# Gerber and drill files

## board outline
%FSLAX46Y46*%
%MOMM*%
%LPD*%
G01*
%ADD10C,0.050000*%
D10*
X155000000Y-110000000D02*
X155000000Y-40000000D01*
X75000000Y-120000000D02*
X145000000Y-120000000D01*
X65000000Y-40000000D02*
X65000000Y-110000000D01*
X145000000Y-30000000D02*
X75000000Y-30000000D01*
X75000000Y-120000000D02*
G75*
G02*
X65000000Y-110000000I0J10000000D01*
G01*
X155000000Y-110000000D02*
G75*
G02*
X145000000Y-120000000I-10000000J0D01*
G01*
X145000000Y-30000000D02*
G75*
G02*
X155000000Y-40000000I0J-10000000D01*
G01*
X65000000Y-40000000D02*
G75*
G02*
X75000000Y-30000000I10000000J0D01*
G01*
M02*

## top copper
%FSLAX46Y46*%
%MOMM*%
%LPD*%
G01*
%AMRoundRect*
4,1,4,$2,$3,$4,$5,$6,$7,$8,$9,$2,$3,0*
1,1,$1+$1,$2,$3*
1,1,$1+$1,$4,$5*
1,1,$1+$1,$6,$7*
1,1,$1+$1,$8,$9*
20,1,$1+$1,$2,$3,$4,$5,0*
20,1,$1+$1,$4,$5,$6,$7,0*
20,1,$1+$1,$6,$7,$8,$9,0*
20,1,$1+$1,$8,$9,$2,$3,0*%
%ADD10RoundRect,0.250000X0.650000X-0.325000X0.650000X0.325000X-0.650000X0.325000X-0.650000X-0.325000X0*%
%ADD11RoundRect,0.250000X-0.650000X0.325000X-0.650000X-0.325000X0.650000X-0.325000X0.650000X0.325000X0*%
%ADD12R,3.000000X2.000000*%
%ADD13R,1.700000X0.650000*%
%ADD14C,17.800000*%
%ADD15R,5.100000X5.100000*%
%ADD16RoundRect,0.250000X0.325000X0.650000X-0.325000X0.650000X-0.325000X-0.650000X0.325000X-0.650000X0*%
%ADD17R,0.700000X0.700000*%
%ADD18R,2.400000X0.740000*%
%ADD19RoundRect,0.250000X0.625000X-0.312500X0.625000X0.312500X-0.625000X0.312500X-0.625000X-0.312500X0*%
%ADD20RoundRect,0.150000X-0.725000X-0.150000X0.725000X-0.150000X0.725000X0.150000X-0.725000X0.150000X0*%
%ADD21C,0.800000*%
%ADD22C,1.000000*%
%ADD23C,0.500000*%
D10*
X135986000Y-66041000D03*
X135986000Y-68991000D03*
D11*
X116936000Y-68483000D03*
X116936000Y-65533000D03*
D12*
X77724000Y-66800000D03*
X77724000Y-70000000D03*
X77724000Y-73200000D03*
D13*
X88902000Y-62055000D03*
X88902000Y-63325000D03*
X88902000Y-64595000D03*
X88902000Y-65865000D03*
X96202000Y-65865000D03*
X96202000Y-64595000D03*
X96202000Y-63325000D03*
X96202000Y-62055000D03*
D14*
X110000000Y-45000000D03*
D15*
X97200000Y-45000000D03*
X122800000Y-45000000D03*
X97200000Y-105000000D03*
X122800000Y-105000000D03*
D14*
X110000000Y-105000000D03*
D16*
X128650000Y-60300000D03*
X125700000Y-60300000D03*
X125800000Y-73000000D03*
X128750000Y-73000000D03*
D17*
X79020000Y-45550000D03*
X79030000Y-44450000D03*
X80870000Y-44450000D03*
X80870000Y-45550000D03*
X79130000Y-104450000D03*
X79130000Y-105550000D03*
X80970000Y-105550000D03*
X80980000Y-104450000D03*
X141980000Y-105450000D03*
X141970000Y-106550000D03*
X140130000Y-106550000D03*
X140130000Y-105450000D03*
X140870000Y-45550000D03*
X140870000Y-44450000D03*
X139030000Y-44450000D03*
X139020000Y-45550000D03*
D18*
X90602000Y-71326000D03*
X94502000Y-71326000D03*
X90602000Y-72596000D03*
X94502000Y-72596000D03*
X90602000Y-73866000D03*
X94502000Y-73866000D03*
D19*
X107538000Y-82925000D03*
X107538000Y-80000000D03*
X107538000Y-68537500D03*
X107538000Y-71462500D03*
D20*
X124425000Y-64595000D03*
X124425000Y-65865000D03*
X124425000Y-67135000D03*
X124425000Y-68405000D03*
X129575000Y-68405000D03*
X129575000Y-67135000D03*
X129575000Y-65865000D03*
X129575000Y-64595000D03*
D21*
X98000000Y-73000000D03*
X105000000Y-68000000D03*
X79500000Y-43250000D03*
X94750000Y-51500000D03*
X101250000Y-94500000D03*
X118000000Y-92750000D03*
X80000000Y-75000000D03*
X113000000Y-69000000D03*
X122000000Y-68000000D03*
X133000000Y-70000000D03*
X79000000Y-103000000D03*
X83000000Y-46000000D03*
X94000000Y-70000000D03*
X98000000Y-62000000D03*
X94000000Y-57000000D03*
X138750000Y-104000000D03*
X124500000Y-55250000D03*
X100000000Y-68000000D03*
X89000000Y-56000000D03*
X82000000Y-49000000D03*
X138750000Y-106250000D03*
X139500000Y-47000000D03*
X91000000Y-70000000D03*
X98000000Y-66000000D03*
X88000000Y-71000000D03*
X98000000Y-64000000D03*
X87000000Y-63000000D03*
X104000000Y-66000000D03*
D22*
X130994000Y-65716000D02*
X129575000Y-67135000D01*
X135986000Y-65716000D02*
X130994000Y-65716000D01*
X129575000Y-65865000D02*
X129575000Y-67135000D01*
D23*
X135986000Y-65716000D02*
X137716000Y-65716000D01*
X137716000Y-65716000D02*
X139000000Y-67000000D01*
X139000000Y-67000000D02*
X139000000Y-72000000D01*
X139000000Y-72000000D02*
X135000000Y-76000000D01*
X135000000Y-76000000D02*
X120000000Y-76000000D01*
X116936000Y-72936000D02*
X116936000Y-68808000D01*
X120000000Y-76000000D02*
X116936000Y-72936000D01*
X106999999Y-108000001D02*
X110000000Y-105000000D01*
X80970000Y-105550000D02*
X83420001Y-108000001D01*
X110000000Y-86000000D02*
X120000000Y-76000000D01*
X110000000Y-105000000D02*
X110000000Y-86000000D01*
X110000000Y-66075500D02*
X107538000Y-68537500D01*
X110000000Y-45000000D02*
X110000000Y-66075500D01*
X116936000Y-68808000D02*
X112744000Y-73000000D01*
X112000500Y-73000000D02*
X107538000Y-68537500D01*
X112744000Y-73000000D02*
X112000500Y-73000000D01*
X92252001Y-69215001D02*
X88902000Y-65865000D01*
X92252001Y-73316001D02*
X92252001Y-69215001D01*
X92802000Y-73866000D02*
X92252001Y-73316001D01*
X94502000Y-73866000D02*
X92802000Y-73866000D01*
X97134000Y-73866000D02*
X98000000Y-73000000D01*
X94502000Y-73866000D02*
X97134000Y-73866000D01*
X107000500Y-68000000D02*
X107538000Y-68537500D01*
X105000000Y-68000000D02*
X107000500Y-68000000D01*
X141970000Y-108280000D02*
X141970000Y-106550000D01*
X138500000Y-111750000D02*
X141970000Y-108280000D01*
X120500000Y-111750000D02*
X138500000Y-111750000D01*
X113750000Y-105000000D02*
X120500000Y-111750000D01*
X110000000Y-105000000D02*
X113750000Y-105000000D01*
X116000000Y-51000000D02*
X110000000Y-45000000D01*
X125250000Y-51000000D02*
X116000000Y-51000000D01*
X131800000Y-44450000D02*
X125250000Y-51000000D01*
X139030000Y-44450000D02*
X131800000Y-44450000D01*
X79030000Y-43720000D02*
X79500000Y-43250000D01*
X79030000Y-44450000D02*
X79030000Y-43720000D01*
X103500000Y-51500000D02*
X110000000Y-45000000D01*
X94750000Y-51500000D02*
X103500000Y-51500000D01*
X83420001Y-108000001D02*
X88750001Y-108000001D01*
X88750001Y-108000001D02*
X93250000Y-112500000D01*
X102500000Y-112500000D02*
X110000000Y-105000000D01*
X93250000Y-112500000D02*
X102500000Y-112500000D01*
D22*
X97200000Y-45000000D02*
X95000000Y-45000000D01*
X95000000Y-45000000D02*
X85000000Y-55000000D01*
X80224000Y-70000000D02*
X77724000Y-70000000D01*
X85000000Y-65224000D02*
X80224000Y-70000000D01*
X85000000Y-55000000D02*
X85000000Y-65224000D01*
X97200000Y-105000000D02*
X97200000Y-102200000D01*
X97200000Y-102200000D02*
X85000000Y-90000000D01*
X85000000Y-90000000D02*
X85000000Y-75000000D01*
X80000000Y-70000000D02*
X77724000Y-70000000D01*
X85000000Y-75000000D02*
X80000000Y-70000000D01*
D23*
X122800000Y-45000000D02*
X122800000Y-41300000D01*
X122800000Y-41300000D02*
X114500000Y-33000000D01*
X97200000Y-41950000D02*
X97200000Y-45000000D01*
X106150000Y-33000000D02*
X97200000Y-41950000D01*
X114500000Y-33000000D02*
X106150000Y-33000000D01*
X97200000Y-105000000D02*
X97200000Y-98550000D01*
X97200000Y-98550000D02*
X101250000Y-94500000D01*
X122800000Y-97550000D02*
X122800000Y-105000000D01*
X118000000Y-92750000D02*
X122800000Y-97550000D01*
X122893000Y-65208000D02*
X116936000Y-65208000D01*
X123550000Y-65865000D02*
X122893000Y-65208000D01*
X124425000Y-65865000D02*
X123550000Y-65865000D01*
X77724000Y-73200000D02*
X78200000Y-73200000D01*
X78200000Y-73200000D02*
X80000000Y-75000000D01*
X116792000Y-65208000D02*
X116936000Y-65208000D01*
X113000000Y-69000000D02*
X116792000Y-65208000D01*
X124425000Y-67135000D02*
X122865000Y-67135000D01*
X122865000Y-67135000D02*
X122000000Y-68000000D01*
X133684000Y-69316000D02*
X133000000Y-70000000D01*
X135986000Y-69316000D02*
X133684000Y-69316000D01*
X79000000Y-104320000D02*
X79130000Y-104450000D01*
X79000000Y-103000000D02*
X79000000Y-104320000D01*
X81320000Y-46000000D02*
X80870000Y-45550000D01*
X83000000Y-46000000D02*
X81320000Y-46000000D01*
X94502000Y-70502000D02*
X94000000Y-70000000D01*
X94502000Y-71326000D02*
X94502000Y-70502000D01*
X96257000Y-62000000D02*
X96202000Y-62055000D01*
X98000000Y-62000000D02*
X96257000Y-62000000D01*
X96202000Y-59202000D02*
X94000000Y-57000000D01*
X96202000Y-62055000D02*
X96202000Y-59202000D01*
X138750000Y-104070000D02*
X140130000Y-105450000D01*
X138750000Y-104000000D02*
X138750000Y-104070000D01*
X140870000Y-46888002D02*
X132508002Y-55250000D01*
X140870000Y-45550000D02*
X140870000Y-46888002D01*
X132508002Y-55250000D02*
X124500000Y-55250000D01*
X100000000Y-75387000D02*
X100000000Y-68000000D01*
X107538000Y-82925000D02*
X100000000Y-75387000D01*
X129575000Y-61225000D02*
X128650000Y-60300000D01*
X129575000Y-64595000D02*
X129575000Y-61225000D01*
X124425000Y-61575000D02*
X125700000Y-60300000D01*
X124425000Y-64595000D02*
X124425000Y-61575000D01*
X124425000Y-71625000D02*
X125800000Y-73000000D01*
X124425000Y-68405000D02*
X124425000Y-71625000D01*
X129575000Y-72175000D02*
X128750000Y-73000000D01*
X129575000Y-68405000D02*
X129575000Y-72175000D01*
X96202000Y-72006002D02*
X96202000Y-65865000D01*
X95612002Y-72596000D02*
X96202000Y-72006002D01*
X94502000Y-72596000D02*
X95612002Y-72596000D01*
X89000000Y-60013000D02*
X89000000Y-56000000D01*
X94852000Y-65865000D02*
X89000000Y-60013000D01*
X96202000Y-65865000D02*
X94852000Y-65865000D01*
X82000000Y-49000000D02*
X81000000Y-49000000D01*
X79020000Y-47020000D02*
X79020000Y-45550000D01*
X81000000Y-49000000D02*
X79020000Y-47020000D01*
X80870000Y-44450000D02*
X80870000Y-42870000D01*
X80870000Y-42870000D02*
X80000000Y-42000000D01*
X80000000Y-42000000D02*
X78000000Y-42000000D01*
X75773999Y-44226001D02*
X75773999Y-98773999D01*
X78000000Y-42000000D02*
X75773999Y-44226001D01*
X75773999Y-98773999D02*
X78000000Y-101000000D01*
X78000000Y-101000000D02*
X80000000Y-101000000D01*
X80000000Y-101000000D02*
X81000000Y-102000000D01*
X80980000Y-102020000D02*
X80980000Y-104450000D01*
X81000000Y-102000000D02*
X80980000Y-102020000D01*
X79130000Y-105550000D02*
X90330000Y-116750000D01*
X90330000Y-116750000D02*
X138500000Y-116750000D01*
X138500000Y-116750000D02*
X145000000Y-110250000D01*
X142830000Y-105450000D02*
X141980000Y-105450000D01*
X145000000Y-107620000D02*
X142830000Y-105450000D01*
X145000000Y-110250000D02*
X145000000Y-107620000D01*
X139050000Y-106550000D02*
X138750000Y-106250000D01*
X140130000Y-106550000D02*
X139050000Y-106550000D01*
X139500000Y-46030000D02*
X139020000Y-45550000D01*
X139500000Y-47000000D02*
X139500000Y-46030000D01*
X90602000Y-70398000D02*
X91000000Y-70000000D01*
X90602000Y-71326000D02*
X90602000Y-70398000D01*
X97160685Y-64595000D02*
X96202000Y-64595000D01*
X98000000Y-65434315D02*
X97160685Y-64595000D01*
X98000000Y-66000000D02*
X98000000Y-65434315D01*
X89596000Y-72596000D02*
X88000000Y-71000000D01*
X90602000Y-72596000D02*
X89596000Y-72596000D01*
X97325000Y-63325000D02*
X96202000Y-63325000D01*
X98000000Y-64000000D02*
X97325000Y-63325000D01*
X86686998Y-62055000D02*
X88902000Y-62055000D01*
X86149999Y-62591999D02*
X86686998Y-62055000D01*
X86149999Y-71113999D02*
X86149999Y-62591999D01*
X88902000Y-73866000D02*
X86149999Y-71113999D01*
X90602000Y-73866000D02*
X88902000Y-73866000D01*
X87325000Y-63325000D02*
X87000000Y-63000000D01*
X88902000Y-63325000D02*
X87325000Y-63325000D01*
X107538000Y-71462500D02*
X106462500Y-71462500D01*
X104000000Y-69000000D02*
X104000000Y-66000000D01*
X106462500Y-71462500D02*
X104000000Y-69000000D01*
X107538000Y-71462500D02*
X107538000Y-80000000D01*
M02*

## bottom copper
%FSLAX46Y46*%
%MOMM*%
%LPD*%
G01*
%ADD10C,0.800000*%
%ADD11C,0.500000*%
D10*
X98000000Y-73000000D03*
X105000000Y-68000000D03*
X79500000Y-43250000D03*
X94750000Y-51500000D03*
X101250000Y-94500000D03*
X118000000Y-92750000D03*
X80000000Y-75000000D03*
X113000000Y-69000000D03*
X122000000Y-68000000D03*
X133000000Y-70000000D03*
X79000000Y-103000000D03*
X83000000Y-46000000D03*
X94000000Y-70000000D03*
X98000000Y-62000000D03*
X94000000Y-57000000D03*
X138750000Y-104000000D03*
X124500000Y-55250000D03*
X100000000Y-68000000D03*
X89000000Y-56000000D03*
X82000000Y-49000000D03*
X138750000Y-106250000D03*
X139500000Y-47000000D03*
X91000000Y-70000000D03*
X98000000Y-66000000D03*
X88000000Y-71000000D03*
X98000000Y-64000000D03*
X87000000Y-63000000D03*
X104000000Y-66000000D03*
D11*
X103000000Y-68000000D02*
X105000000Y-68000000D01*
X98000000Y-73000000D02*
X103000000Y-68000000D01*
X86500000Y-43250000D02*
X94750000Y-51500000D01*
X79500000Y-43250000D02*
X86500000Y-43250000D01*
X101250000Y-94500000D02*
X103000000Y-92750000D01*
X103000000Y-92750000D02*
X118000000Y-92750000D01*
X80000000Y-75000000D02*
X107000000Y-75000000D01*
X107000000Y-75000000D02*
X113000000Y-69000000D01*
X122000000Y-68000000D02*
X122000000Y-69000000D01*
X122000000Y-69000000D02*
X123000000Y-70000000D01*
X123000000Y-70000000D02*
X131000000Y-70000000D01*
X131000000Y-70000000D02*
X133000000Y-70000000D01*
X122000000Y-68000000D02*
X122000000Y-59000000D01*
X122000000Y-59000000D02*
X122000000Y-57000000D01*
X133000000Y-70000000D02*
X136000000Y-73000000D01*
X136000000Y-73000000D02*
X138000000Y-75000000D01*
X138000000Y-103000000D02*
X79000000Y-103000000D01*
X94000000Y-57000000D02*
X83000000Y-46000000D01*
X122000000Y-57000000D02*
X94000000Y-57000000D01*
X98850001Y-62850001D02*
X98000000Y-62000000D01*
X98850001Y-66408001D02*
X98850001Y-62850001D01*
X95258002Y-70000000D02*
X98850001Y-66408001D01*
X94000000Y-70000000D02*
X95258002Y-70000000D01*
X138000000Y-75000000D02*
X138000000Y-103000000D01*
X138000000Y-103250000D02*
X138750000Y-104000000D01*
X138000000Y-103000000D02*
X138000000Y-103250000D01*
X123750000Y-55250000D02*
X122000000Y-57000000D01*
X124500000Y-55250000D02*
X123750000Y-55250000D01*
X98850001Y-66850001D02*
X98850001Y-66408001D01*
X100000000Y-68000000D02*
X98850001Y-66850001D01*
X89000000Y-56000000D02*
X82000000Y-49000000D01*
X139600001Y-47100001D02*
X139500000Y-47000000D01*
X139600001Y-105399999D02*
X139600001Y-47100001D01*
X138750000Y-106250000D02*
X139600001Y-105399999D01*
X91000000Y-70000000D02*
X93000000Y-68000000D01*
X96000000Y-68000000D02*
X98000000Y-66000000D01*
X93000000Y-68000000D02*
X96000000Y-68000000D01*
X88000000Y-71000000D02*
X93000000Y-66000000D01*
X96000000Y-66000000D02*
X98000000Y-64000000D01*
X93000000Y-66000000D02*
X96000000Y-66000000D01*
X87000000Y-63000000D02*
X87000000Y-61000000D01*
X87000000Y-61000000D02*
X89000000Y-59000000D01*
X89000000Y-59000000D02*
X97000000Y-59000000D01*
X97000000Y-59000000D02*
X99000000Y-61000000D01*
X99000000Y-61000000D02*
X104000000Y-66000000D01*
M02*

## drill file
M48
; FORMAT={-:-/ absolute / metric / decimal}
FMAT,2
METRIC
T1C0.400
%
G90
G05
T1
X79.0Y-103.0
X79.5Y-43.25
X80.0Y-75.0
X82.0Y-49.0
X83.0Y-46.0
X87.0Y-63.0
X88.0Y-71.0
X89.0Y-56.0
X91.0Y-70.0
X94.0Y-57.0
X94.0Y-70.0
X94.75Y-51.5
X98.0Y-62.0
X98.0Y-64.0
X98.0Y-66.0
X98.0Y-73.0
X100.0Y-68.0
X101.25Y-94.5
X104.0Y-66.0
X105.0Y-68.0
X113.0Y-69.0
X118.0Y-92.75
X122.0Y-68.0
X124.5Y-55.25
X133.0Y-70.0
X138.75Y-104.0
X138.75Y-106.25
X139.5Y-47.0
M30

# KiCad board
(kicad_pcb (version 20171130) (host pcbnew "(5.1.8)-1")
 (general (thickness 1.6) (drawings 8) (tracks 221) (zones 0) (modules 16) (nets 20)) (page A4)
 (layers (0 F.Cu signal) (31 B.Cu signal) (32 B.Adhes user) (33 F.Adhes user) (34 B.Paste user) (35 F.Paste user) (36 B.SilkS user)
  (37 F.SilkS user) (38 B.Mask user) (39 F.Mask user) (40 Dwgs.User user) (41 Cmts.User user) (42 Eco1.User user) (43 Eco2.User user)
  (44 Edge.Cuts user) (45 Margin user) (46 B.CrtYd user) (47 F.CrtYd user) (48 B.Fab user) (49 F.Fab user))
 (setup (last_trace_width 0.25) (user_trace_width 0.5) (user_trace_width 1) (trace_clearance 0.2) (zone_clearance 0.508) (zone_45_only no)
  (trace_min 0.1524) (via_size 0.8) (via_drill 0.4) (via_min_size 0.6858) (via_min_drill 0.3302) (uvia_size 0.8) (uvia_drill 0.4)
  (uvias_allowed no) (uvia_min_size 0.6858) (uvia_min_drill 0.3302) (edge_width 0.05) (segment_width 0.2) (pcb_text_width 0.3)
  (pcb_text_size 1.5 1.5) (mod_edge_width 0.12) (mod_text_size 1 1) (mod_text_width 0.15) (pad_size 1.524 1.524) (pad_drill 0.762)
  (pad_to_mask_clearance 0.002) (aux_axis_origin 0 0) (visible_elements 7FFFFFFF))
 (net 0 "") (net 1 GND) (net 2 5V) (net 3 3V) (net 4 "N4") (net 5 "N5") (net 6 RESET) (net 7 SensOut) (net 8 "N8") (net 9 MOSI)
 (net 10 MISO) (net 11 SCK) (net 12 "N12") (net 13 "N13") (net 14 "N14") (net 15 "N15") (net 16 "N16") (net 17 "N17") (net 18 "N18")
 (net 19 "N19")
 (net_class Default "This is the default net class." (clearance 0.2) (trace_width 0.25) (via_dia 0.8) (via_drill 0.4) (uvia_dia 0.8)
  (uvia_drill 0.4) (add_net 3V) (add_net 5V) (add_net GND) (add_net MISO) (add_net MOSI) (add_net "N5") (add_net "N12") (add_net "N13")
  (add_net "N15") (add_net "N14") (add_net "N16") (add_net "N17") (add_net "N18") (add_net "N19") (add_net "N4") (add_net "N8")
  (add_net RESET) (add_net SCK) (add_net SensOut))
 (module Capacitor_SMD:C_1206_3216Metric (layer F.Cu) (at 135.986 67.516 90)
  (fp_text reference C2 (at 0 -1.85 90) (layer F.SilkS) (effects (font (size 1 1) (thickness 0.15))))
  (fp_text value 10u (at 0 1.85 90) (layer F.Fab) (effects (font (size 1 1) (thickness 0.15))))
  (pad 2 smd roundrect (at 1.475 0 90) (size 1.15 1.8) (layers F.Cu F.Paste F.Mask) (roundrect_rratio 0.217391) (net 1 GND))
  (pad 1 smd roundrect (at -1.475 0 90) (size 1.15 1.8) (layers F.Cu F.Paste F.Mask) (roundrect_rratio 0.217391) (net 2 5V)))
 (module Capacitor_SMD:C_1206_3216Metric (layer F.Cu) (at 116.936 67.008 270)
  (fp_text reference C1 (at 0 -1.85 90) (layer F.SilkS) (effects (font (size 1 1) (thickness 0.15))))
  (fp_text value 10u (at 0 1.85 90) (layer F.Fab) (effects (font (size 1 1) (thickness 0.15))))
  (pad 2 smd roundrect (at 1.475 0 270) (size 1.15 1.8) (layers F.Cu F.Paste F.Mask) (roundrect_rratio 0.217391) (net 1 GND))
  (pad 1 smd roundrect (at -1.475 0 270) (size 1.15 1.8) (layers F.Cu F.Paste F.Mask) (roundrect_rratio 0.217391) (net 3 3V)))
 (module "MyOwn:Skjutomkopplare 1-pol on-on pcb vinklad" (layer F.Cu) (at 77.724 70 90)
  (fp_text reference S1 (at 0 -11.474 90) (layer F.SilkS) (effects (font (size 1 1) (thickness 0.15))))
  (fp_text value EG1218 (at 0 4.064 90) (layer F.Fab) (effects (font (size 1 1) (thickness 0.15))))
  (pad 3 smd rect (at 3.2 0 180) (size 3 2) (layers F.Cu F.Paste F.Mask) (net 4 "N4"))
  (pad 2 smd rect (at 0 0 180) (size 3 2) (layers F.Cu F.Paste F.Mask) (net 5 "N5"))
  (pad 1 smd rect (at -3.2 0 180) (size 3 2) (layers F.Cu F.Paste F.Mask) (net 3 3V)))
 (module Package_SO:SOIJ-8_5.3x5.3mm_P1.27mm (layer F.Cu) (at 92.552 63.96)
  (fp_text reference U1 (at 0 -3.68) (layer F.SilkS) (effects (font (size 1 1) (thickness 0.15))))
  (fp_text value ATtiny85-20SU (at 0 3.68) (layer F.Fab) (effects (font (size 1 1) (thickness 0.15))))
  (pad 1 smd rect (at -3.65 -1.905) (size 1.7 0.65) (layers F.Cu F.Paste F.Mask) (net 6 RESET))
  (pad 2 smd rect (at -3.65 -0.635) (size 1.7 0.65) (layers F.Cu F.Paste F.Mask) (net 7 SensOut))
  (pad 3 smd rect (at -3.65 0.635) (size 1.7 0.65) (layers F.Cu F.Paste F.Mask) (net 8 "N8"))
  (pad 4 smd rect (at -3.65 1.905) (size 1.7 0.65) (layers F.Cu F.Paste F.Mask) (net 1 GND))
  (pad 5 smd rect (at 3.65 1.905) (size 1.7 0.65) (layers F.Cu F.Paste F.Mask) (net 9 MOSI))
  (pad 6 smd rect (at 3.65 0.635) (size 1.7 0.65) (layers F.Cu F.Paste F.Mask) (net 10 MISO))
  (pad 7 smd rect (at 3.65 -0.635) (size 1.7 0.65) (layers F.Cu F.Paste F.Mask) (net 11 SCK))
  (pad 8 smd rect (at 3.65 -1.905) (size 1.7 0.65) (layers F.Cu F.Paste F.Mask) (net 2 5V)))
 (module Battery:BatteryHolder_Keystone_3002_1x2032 (layer F.Cu) (at 110 45)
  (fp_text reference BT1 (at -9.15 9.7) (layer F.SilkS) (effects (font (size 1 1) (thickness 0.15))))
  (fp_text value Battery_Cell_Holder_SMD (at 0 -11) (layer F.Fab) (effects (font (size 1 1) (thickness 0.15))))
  (pad 2 smd circle (at 0 0) (size 17.8 17.8) (layers F.Cu F.Mask) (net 1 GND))
  (pad 1 smd rect (at -12.8 0) (size 5.1 5.1) (layers F.Cu F.Paste F.Mask) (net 5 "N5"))
  (pad 1 smd rect (at 12.8 0) (size 5.1 5.1) (layers F.Cu F.Paste F.Mask) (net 5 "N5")))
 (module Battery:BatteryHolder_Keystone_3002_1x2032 (layer F.Cu) (at 110 105 180)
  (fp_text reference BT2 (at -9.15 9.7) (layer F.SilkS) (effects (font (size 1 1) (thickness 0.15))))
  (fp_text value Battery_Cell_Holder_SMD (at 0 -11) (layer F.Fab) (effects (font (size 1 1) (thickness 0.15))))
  (pad 1 smd rect (at 12.8 0 180) (size 5.1 5.1) (layers F.Cu F.Paste F.Mask) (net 5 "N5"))
  (pad 1 smd rect (at -12.8 0 180) (size 5.1 5.1) (layers F.Cu F.Paste F.Mask) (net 5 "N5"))
  (pad 2 smd circle (at 0 0 180) (size 17.8 17.8) (layers F.Cu F.Mask) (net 1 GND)))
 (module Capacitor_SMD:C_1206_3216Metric (layer F.Cu) (at 127.175 60.3 180)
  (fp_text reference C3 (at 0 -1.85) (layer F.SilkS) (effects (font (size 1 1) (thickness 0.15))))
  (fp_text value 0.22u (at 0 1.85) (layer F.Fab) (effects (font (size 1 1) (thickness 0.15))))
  (pad 1 smd roundrect (at -1.475 0 180) (size 1.15 1.8) (layers F.Cu F.Paste F.Mask) (roundrect_rratio 0.217391) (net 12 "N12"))
  (pad 2 smd roundrect (at 1.475 0 180) (size 1.15 1.8) (layers F.Cu F.Paste F.Mask) (roundrect_rratio 0.217391) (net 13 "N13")))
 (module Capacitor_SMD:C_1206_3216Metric (layer F.Cu) (at 127.275 73 180)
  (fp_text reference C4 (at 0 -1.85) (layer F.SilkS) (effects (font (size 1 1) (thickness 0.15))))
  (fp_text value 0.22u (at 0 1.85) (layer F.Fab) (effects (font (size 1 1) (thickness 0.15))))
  (pad 2 smd roundrect (at 1.475 0 180) (size 1.15 1.8) (layers F.Cu F.Paste F.Mask) (roundrect_rratio 0.217391) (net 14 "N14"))
  (pad 1 smd roundrect (at -1.475 0 180) (size 1.15 1.8) (layers F.Cu F.Paste F.Mask) (roundrect_rratio 0.217391) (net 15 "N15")))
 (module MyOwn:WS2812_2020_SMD (layer F.Cu) (at 80 45)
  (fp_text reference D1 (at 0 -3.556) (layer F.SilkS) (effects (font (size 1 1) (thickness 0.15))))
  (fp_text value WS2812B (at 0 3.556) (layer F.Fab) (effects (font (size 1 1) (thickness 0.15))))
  (pad 4 smd rect (at -0.98 0.55) (size 0.7 0.7) (layers F.Cu F.Paste F.Mask) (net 9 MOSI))
  (pad 3 smd rect (at -0.97 -0.55) (size 0.7 0.7) (layers F.Cu F.Paste F.Mask) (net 1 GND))
  (pad 2 smd rect (at 0.87 -0.55) (size 0.7 0.7) (layers F.Cu F.Paste F.Mask) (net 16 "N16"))
  (pad 1 smd rect (at 0.87 0.55) (size 0.7 0.7) (layers F.Cu F.Paste F.Mask) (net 2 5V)))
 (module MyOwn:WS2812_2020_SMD (layer F.Cu) (at 80 105 180)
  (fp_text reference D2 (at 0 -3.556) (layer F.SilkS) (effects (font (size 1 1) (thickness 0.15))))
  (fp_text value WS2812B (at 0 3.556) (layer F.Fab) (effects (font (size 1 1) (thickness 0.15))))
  (pad 1 smd rect (at 0.87 0.55 180) (size 0.7 0.7) (layers F.Cu F.Paste F.Mask) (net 2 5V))
  (pad 2 smd rect (at 0.87 -0.55 180) (size 0.7 0.7) (layers F.Cu F.Paste F.Mask) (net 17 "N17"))
  (pad 3 smd rect (at -0.97 -0.55 180) (size 0.7 0.7) (layers F.Cu F.Paste F.Mask) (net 1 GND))
  (pad 4 smd rect (at -0.98 0.55 180) (size 0.7 0.7) (layers F.Cu F.Paste F.Mask) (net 16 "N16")))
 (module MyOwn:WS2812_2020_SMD (layer F.Cu) (at 141 106 180)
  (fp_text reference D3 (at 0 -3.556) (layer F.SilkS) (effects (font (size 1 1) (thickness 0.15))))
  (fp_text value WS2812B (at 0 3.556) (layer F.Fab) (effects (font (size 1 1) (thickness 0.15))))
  (pad 4 smd rect (at -0.98 0.55 180) (size 0.7 0.7) (layers F.Cu F.Paste F.Mask) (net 17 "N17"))
  (pad 3 smd rect (at -0.97 -0.55 180) (size 0.7 0.7) (layers F.Cu F.Paste F.Mask) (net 1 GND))
  (pad 2 smd rect (at 0.87 -0.55 180) (size 0.7 0.7) (layers F.Cu F.Paste F.Mask) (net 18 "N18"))
  (pad 1 smd rect (at 0.87 0.55 180) (size 0.7 0.7) (layers F.Cu F.Paste F.Mask) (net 2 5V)))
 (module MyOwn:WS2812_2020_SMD (layer F.Cu) (at 140 45)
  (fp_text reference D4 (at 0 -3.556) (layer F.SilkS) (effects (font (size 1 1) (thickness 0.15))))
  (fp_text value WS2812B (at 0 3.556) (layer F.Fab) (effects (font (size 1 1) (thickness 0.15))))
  (pad 1 smd rect (at 0.87 0.55) (size 0.7 0.7) (layers F.Cu F.Paste F.Mask) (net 2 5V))
  (pad 2 smd rect (at 0.87 -0.55) (size 0.7 0.7) (layers F.Cu F.Paste F.Mask) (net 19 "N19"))
  (pad 3 smd rect (at -0.97 -0.55) (size 0.7 0.7) (layers F.Cu F.Paste F.Mask) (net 1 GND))
  (pad 4 smd rect (at -0.98 0.55) (size 0.7 0.7) (layers F.Cu F.Paste F.Mask) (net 18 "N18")))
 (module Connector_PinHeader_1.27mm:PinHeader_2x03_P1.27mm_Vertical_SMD (layer F.Cu) (at 92.552 72.596)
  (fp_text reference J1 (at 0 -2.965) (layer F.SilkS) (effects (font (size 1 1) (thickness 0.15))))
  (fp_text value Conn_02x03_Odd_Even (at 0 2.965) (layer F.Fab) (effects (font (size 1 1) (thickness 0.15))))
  (pad 1 smd rect (at -1.95 -1.27) (size 2.4 0.74) (layers F.Cu F.Paste F.Mask) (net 10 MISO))
  (pad 2 smd rect (at 1.95 -1.27) (size 2.4 0.74) (layers F.Cu F.Paste F.Mask) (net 2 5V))
  (pad 3 smd rect (at -1.95 0) (size 2.4 0.74) (layers F.Cu F.Paste F.Mask) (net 11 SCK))
  (pad 4 smd rect (at 1.95 0) (size 2.4 0.74) (layers F.Cu F.Paste F.Mask) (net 9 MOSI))
  (pad 5 smd rect (at -1.95 1.27) (size 2.4 0.74) (layers F.Cu F.Paste F.Mask) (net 6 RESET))
  (pad 6 smd rect (at 1.95 1.27) (size 2.4 0.74) (layers F.Cu F.Paste F.Mask) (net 1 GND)))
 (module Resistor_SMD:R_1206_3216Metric (layer F.Cu) (at 107.538 81.4625 90)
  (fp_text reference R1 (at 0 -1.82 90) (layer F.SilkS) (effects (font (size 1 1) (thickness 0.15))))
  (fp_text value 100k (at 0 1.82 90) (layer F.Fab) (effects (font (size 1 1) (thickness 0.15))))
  (pad 1 smd roundrect (at -1.4625 0 90) (size 1.125 1.75) (layers F.Cu F.Paste F.Mask) (roundrect_rratio 0.222222) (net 2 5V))
  (pad 2 smd roundrect (at 1.4625 0 90) (size 1.125 1.75) (layers F.Cu F.Paste F.Mask) (roundrect_rratio 0.222222) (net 7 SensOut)))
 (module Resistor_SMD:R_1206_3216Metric (layer F.Cu) (at 107.538 70 90)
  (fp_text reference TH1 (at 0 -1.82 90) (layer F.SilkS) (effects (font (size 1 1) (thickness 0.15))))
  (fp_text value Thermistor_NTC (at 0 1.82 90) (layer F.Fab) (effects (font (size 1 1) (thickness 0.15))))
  (pad 2 smd roundrect (at 1.4625 0 90) (size 1.125 1.75) (layers F.Cu F.Paste F.Mask) (roundrect_rratio 0.222222) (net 1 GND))
  (pad 1 smd roundrect (at -1.4625 0 90) (size 1.125 1.75) (layers F.Cu F.Paste F.Mask) (roundrect_rratio 0.222222) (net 7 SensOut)))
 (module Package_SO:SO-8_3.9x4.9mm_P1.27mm (layer F.Cu) (at 127 66.5)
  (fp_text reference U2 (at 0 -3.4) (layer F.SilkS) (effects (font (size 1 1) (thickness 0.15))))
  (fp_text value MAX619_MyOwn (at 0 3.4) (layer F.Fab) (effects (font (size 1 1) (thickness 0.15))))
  (pad 1 smd roundrect (at -2.575 -1.905) (size 1.75 0.6) (layers F.Cu F.Paste F.Mask) (roundrect_rratio 0.25) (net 13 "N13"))
  (pad 2 smd roundrect (at -2.575 -0.635) (size 1.75 0.6) (layers F.Cu F.Paste F.Mask) (roundrect_rratio 0.25) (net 3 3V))
  (pad 3 smd roundrect (at -2.575 0.635) (size 1.75 0.6) (layers F.Cu F.Paste F.Mask) (roundrect_rratio 0.25) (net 2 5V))
  (pad 4 smd roundrect (at -2.575 1.905) (size 1.75 0.6) (layers F.Cu F.Paste F.Mask) (roundrect_rratio 0.25) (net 14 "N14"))
  (pad 5 smd roundrect (at 2.575 1.905) (size 1.75 0.6) (layers F.Cu F.Paste F.Mask) (roundrect_rratio 0.25) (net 15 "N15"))
  (pad 6 smd roundrect (at 2.575 0.635) (size 1.75 0.6) (layers F.Cu F.Paste F.Mask) (roundrect_rratio 0.25) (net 1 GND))
  (pad 7 smd roundrect (at 2.575 -0.635) (size 1.75 0.6) (layers F.Cu F.Paste F.Mask) (roundrect_rratio 0.25) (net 1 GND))
  (pad 8 smd roundrect (at 2.575 -1.905) (size 1.75 0.6) (layers F.Cu F.Paste F.Mask) (roundrect_rratio 0.25) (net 12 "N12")))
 (gr_line (start 155 110) (end 155 40) (layer Edge.Cuts) (width 0.05))
 (gr_line (start 75 120) (end 145 120) (layer Edge.Cuts) (width 0.05))
 (gr_line (start 65 40) (end 65 110) (layer Edge.Cuts) (width 0.05))
 (gr_line (start 145 30) (end 75 30) (layer Edge.Cuts) (width 0.05))
 (gr_arc (start 75 110) (end 65 110) (angle -90) (layer Edge.Cuts) (width 0.05))
 (gr_arc (start 145 110) (end 145 120) (angle -90) (layer Edge.Cuts) (width 0.05))
 (gr_arc (start 145 40) (end 155 40) (angle -90) (layer Edge.Cuts) (width 0.05))
 (gr_arc (start 75 40) (end 75 30) (angle -90) (layer Edge.Cuts) (width 0.05))
 (segment (start 130.994 65.716) (end 129.575 67.135) (width 1) (layer F.Cu) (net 1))
 (segment (start 135.986 65.716) (end 130.994 65.716) (width 1) (layer F.Cu) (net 1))
 (segment (start 129.575 65.865) (end 129.575 67.135) (width 1) (layer F.Cu) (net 1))
 (segment (start 135.986 65.716) (end 137.716 65.716) (width 0.5) (layer F.Cu) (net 1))
 (segment (start 137.716 65.716) (end 139 67) (width 0.5) (layer F.Cu) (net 1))
 (segment (start 139 67) (end 139 72) (width 0.5) (layer F.Cu) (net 1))
 (segment (start 139 72) (end 135 76) (width 0.5) (layer F.Cu) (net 1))
 (segment (start 135 76) (end 120 76) (width 0.5) (layer F.Cu) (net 1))
 (segment (start 116.936 72.936) (end 116.936 68.808) (width 0.5) (layer F.Cu) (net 1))
 (segment (start 120 76) (end 116.936 72.936) (width 0.5) (layer F.Cu) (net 1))
 (segment (start 106.999999 108.000001) (end 110 105) (width 0.5) (layer F.Cu) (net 1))
 (segment (start 80.97 105.55) (end 83.420001 108.000001) (width 0.5) (layer F.Cu) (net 1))
 (segment (start 110 86) (end 120 76) (width 0.5) (layer F.Cu) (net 1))
 (segment (start 110 105) (end 110 86) (width 0.5) (layer F.Cu) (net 1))
 (segment (start 110 66.0755) (end 107.538 68.5375) (width 0.5) (layer F.Cu) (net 1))
 (segment (start 110 45) (end 110 66.0755) (width 0.5) (layer F.Cu) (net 1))
 (segment (start 116.936 68.808) (end 112.744 73) (width 0.5) (layer F.Cu) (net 1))
 (segment (start 112.0005 73) (end 107.538 68.5375) (width 0.5) (layer F.Cu) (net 1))
 (segment (start 112.744 73) (end 112.0005 73) (width 0.5) (layer F.Cu) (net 1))
 (segment (start 92.252001 69.215001) (end 88.902 65.865) (width 0.5) (layer F.Cu) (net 1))
 (segment (start 92.252001 73.316001) (end 92.252001 69.215001) (width 0.5) (layer F.Cu) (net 1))
 (segment (start 92.802 73.866) (end 92.252001 73.316001) (width 0.5) (layer F.Cu) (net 1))
 (segment (start 94.502 73.866) (end 92.802 73.866) (width 0.5) (layer F.Cu) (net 1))
 (via (at 98 73) (size 0.8) (drill 0.4) (layers F.Cu B.Cu) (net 1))
 (segment (start 97.134 73.866) (end 98 73) (width 0.5) (layer F.Cu) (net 1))
 (segment (start 94.502 73.866) (end 97.134 73.866) (width 0.5) (layer F.Cu) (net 1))
 (via (at 105 68) (size 0.8) (drill 0.4) (layers F.Cu B.Cu) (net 1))
 (segment (start 103 68) (end 105 68) (width 0.5) (layer B.Cu) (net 1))
 (segment (start 98 73) (end 103 68) (width 0.5) (layer B.Cu) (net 1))
 (segment (start 107.0005 68) (end 107.538 68.5375) (width 0.5) (layer F.Cu) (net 1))
 (segment (start 105 68) (end 107.0005 68) (width 0.5) (layer F.Cu) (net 1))
 (segment (start 141.97 108.28) (end 141.97 106.55) (width 0.5) (layer F.Cu) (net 1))
 (segment (start 138.5 111.75) (end 141.97 108.28) (width 0.5) (layer F.Cu) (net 1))
 (segment (start 120.5 111.75) (end 138.5 111.75) (width 0.5) (layer F.Cu) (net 1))
 (segment (start 113.75 105) (end 120.5 111.75) (width 0.5) (layer F.Cu) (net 1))
 (segment (start 110 105) (end 113.75 105) (width 0.5) (layer F.Cu) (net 1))
 (segment (start 116 51) (end 110 45) (width 0.5) (layer F.Cu) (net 1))
 (segment (start 125.25 51) (end 116 51) (width 0.5) (layer F.Cu) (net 1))
 (segment (start 131.8 44.45) (end 125.25 51) (width 0.5) (layer F.Cu) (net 1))
 (segment (start 139.03 44.45) (end 131.8 44.45) (width 0.5) (layer F.Cu) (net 1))
 (via (at 79.5 43.25) (size 0.8) (drill 0.4) (layers F.Cu B.Cu) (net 1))
 (segment (start 79.03 43.72) (end 79.5 43.25) (width 0.5) (layer F.Cu) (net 1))
 (segment (start 79.03 44.45) (end 79.03 43.72) (width 0.5) (layer F.Cu) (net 1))
 (via (at 94.75 51.5) (size 0.8) (drill 0.4) (layers F.Cu B.Cu) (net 1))
 (segment (start 86.5 43.25) (end 94.75 51.5) (width 0.5) (layer B.Cu) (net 1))
 (segment (start 79.5 43.25) (end 86.5 43.25) (width 0.5) (layer B.Cu) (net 1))
 (segment (start 103.5 51.5) (end 110 45) (width 0.5) (layer F.Cu) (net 1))
 (segment (start 94.75 51.5) (end 103.5 51.5) (width 0.5) (layer F.Cu) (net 1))
 (segment (start 83.420001 108.000001) (end 88.750001 108.000001) (width 0.5) (layer F.Cu) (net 1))
 (segment (start 88.750001 108.000001) (end 93.25 112.5) (width 0.5) (layer F.Cu) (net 1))
 (segment (start 102.5 112.5) (end 110 105) (width 0.5) (layer F.Cu) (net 1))
 (segment (start 93.25 112.5) (end 102.5 112.5) (width 0.5) (layer F.Cu) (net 1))
 (segment (start 97.2 45) (end 95 45) (width 1) (layer F.Cu) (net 5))
 (segment (start 95 45) (end 85 55) (width 1) (layer F.Cu) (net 5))
 (segment (start 80.224 70) (end 77.724 70) (width 1) (layer F.Cu) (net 5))
 (segment (start 85 65.224) (end 80.224 70) (width 1) (layer F.Cu) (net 5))
 (segment (start 85 55) (end 85 65.224) (width 1) (layer F.Cu) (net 5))
 (segment (start 97.2 105) (end 97.2 102.2) (width 1) (layer F.Cu) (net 5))
 (segment (start 97.2 102.2) (end 85 90) (width 1) (layer F.Cu) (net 5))
 (segment (start 85 90) (end 85 75) (width 1) (layer F.Cu) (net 5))
 (segment (start 80 70) (end 77.724 70) (width 1) (layer F.Cu) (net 5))
 (segment (start 85 75) (end 80 70) (width 1) (layer F.Cu) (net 5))
 (segment (start 122.8 45) (end 122.8 41.3) (width 0.5) (layer F.Cu) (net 5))
 (segment (start 122.8 41.3) (end 114.5 33) (width 0.5) (layer F.Cu) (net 5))
 (segment (start 97.2 41.95) (end 97.2 45) (width 0.5) (layer F.Cu) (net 5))
 (segment (start 106.15 33) (end 97.2 41.95) (width 0.5) (layer F.Cu) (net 5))
 (segment (start 114.5 33) (end 106.15 33) (width 0.5) (layer F.Cu) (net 5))
 (segment (start 97.2 105) (end 97.2 98.55) (width 0.5) (layer F.Cu) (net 5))
 (via (at 101.25 94.5) (size 0.8) (drill 0.4) (layers F.Cu B.Cu) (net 5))
 (segment (start 97.2 98.55) (end 101.25 94.5) (width 0.5) (layer F.Cu) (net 5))
 (segment (start 101.25 94.5) (end 103 92.75) (width 0.5) (layer B.Cu) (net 5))
 (via (at 118 92.75) (size 0.8) (drill 0.4) (layers F.Cu B.Cu) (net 5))
 (segment (start 103 92.75) (end 118 92.75) (width 0.5) (layer B.Cu) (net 5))
 (segment (start 122.8 97.55) (end 122.8 105) (width 0.5) (layer F.Cu) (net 5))
 (segment (start 118 92.75) (end 122.8 97.55) (width 0.5) (layer F.Cu) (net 5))
 (segment (start 122.893 65.208) (end 116.936 65.208) (width 0.5) (layer F.Cu) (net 3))
 (segment (start 123.55 65.865) (end 122.893 65.208) (width 0.5) (layer F.Cu) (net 3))
 (segment (start 124.425 65.865) (end 123.55 65.865) (width 0.5) (layer F.Cu) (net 3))
 (segment (start 77.724 73.2) (end 78.2 73.2) (width 0.5) (layer F.Cu) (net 3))
 (via (at 80 75) (size 0.8) (drill 0.4) (layers F.Cu B.Cu) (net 3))
 (segment (start 78.2 73.2) (end 80 75) (width 0.5) (layer F.Cu) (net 3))
 (segment (start 80 75) (end 107 75) (width 0.5) (layer B.Cu) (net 3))
 (via (at 113 69) (size 0.8) (drill 0.4) (layers F.Cu B.Cu) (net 3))
 (segment (start 107 75) (end 113 69) (width 0.5) (layer B.Cu) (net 3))
 (segment (start 116.792 65.208) (end 116.936 65.208) (width 0.5) (layer F.Cu) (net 3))
 (segment (start 113 69) (end 116.792 65.208) (width 0.5) (layer F.Cu) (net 3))
 (segment (start 124.425 67.135) (end 122.865 67.135) (width 0.5) (layer F.Cu) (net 2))
 (via (at 122 68) (size 0.8) (drill 0.4) (layers F.Cu B.Cu) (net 2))
 (segment (start 122.865 67.135) (end 122 68) (width 0.5) (layer F.Cu) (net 2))
 (segment (start 122 68) (end 122 69) (width 0.5) (layer B.Cu) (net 2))
 (segment (start 122 69) (end 123 70) (width 0.5) (layer B.Cu) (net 2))
 (segment (start 123 70) (end 131 70) (width 0.5) (layer B.Cu) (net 2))
 (segment (start 131 70) (end 133 70) (width 0.5) (layer B.Cu) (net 2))
 (via (at 133 70) (size 0.8) (drill 0.4) (layers F.Cu B.Cu) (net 2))
 (segment (start 133.684 69.316) (end 133 70) (width 0.5) (layer F.Cu) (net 2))
 (segment (start 135.986 69.316) (end 133.684 69.316) (width 0.5) (layer F.Cu) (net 2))
 (segment (start 122 68) (end 122 59) (width 0.5) (layer B.Cu) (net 2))
 (segment (start 122 59) (end 122 57) (width 0.5) (layer B.Cu) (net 2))
 (segment (start 133 70) (end 136 73) (width 0.5) (layer B.Cu) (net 2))
 (segment (start 136 73) (end 138 75) (width 0.5) (layer B.Cu) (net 2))
 (via (at 79 103) (size 0.8) (drill 0.4) (layers F.Cu B.Cu) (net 2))
 (segment (start 138 103) (end 79 103) (width 0.5) (layer B.Cu) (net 2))
 (segment (start 79 104.32) (end 79.13 104.45) (width 0.5) (layer F.Cu) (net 2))
 (segment (start 79 103) (end 79 104.32) (width 0.5) (layer F.Cu) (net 2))
 (via (at 83 46) (size 0.8) (drill 0.4) (layers F.Cu B.Cu) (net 2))
 (segment (start 94 57) (end 83 46) (width 0.5) (layer B.Cu) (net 2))
 (segment (start 122 57) (end 94 57) (width 0.5) (layer B.Cu) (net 2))
 (segment (start 81.32 46) (end 80.87 45.55) (width 0.5) (layer F.Cu) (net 2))
 (segment (start 83 46) (end 81.32 46) (width 0.5) (layer F.Cu) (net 2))
 (via (at 94 70) (size 0.8) (drill 0.4) (layers F.Cu B.Cu) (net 2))
 (segment (start 94.502 70.502) (end 94 70) (width 0.5) (layer F.Cu) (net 2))
 (segment (start 94.502 71.326) (end 94.502 70.502) (width 0.5) (layer F.Cu) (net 2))
 (via (at 98 62) (size 0.8) (drill 0.4) (layers F.Cu B.Cu) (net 2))
 (segment (start 98.850001 62.850001) (end 98 62) (width 0.5) (layer B.Cu) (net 2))
 (segment (start 98.850001 66.408001) (end 98.850001 62.850001) (width 0.5) (layer B.Cu) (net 2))
 (segment (start 95.258002 70) (end 98.850001 66.408001) (width 0.5) (layer B.Cu) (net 2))
 (segment (start 94 70) (end 95.258002 70) (width 0.5) (layer B.Cu) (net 2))
 (segment (start 96.257 62) (end 96.202 62.055) (width 0.5) (layer F.Cu) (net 2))
 (segment (start 98 62) (end 96.257 62) (width 0.5) (layer F.Cu) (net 2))
 (via (at 94 57) (size 0.8) (drill 0.4) (layers F.Cu B.Cu) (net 2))
 (segment (start 96.202 59.202) (end 94 57) (width 0.5) (layer F.Cu) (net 2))
 (segment (start 96.202 62.055) (end 96.202 59.202) (width 0.5) (layer F.Cu) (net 2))
 (segment (start 138 75) (end 138 103) (width 0.5) (layer B.Cu) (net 2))
 (via (at 138.75 104) (size 0.8) (drill 0.4) (layers F.Cu B.Cu) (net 2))
 (segment (start 138 103.25) (end 138.75 104) (width 0.5) (layer B.Cu) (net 2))
 (segment (start 138 103) (end 138 103.25) (width 0.5) (layer B.Cu) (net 2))
 (segment (start 138.75 104.07) (end 140.13 105.45) (width 0.5) (layer F.Cu) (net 2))
 (segment (start 138.75 104) (end 138.75 104.07) (width 0.5) (layer F.Cu) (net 2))
 (segment (start 140.87 46.888002) (end 132.508002 55.25) (width 0.5) (layer F.Cu) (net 2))
 (segment (start 140.87 45.55) (end 140.87 46.888002) (width 0.5) (layer F.Cu) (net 2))
 (via (at 124.5 55.25) (size 0.8) (drill 0.4) (layers F.Cu B.Cu) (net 2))
 (segment (start 132.508002 55.25) (end 124.5 55.25) (width 0.5) (layer F.Cu) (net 2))
 (segment (start 123.75 55.25) (end 122 57) (width 0.5) (layer B.Cu) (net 2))
 (segment (start 124.5 55.25) (end 123.75 55.25) (width 0.5) (layer B.Cu) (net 2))
 (via (at 100 68) (size 0.8) (drill 0.4) (layers F.Cu B.Cu) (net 2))
 (segment (start 100 75.387) (end 100 68) (width 0.5) (layer F.Cu) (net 2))
 (segment (start 107.538 82.925) (end 100 75.387) (width 0.5) (layer F.Cu) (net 2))
 (segment (start 98.850001 66.850001) (end 98.850001 66.408001) (width 0.5) (layer B.Cu) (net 2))
 (segment (start 100 68) (end 98.850001 66.850001) (width 0.5) (layer B.Cu) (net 2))
 (segment (start 129.575 61.225) (end 128.65 60.3) (width 0.5) (layer F.Cu) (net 12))
 (segment (start 129.575 64.595) (end 129.575 61.225) (width 0.5) (layer F.Cu) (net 12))
 (segment (start 124.425 61.575) (end 125.7 60.3) (width 0.5) (layer F.Cu) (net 13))
 (segment (start 124.425 64.595) (end 124.425 61.575) (width 0.5) (layer F.Cu) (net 13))
 (segment (start 124.425 71.625) (end 125.8 73) (width 0.5) (layer F.Cu) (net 14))
 (segment (start 124.425 68.405) (end 124.425 71.625) (width 0.5) (layer F.Cu) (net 14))
 (segment (start 129.575 72.175) (end 128.75 73) (width 0.5) (layer F.Cu) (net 15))
 (segment (start 129.575 68.405) (end 129.575 72.175) (width 0.5) (layer F.Cu) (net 15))
 (segment (start 96.202 72.006002) (end 96.202 65.865) (width 0.5) (layer F.Cu) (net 9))
 (segment (start 95.612002 72.596) (end 96.202 72.006002) (width 0.5) (layer F.Cu) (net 9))
 (segment (start 94.502 72.596) (end 95.612002 72.596) (width 0.5) (layer F.Cu) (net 9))
 (via (at 89 56) (size 0.8) (drill 0.4) (layers F.Cu B.Cu) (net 9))
 (segment (start 89 60.013) (end 89 56) (width 0.5) (layer F.Cu) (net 9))
 (segment (start 94.852 65.865) (end 89 60.013) (width 0.5) (layer F.Cu) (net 9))
 (segment (start 96.202 65.865) (end 94.852 65.865) (width 0.5) (layer F.Cu) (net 9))
 (via (at 82 49) (size 0.8) (drill 0.4) (layers F.Cu B.Cu) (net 9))
 (segment (start 89 56) (end 82 49) (width 0.5) (layer B.Cu) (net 9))
 (segment (start 82 49) (end 81 49) (width 0.5) (layer F.Cu) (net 9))
 (segment (start 79.02 47.02) (end 79.02 45.55) (width 0.5) (layer F.Cu) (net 9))
 (segment (start 81 49) (end 79.02 47.02) (width 0.5) (layer F.Cu) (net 9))
 (segment (start 80.87 44.45) (end 80.87 42.87) (width 0.5) (layer F.Cu) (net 16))
 (segment (start 80.87 42.87) (end 80 42) (width 0.5) (layer F.Cu) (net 16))
 (segment (start 80 42) (end 78 42) (width 0.5) (layer F.Cu) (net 16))
 (segment (start 75.773999 44.226001) (end 75.773999 98.773999) (width 0.5) (layer F.Cu) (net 16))
 (segment (start 78 42) (end 75.773999 44.226001) (width 0.5) (layer F.Cu) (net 16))
 (segment (start 75.773999 98.773999) (end 78 101) (width 0.5) (layer F.Cu) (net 16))
 (segment (start 78 101) (end 80 101) (width 0.5) (layer F.Cu) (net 16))
 (segment (start 80 101) (end 81 102) (width 0.5) (layer F.Cu) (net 16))
 (segment (start 80.98 102.02) (end 80.98 104.45) (width 0.5) (layer F.Cu) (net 16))
 (segment (start 81 102) (end 80.98 102.02) (width 0.5) (layer F.Cu) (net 16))
 (segment (start 79.13 105.55) (end 90.33 116.75) (width 0.5) (layer F.Cu) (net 17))
 (segment (start 90.33 116.75) (end 138.5 116.75) (width 0.5) (layer F.Cu) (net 17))
 (segment (start 138.5 116.75) (end 145 110.25) (width 0.5) (layer F.Cu) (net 17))
 (segment (start 142.83 105.45) (end 141.98 105.45) (width 0.5) (layer F.Cu) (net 17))
 (segment (start 145 107.62) (end 142.83 105.45) (width 0.5) (layer F.Cu) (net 17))
 (segment (start 145 110.25) (end 145 107.62) (width 0.5) (layer F.Cu) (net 17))
 (via (at 138.75 106.25) (size 0.8) (drill 0.4) (layers F.Cu B.Cu) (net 18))
 (segment (start 139.05 106.55) (end 138.75 106.25) (width 0.5) (layer F.Cu) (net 18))
 (segment (start 140.13 106.55) (end 139.05 106.55) (width 0.5) (layer F.Cu) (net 18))
 (via (at 139.5 47) (size 0.8) (drill 0.4) (layers F.Cu B.Cu) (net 18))
 (segment (start 139.600001 47.100001) (end 139.5 47) (width 0.5) (layer B.Cu) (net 18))
 (segment (start 139.600001 105.399999) (end 139.600001 47.100001) (width 0.5) (layer B.Cu) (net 18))
 (segment (start 138.75 106.25) (end 139.600001 105.399999) (width 0.5) (layer B.Cu) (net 18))
 (segment (start 139.5 46.03) (end 139.02 45.55) (width 0.5) (layer F.Cu) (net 18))
 (segment (start 139.5 47) (end 139.5 46.03) (width 0.5) (layer F.Cu) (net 18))
 (via (at 91 70) (size 0.8) (drill 0.4) (layers F.Cu B.Cu) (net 10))
 (segment (start 90.602 70.398) (end 91 70) (width 0.5) (layer F.Cu) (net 10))
 (segment (start 90.602 71.326) (end 90.602 70.398) (width 0.5) (layer F.Cu) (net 10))
 (segment (start 91 70) (end 93 68) (width 0.5) (layer B.Cu) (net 10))
 (via (at 98 66) (size 0.8) (drill 0.4) (layers F.Cu B.Cu) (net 10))
 (segment (start 96 68) (end 98 66) (width 0.5) (layer B.Cu) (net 10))
 (segment (start 93 68) (end 96 68) (width 0.5) (layer B.Cu) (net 10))
 (segment (start 97.160685 64.595) (end 96.202 64.595) (width 0.5) (layer F.Cu) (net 10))
 (segment (start 98 65.434315) (end 97.160685 64.595) (width 0.5) (layer F.Cu) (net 10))
 (segment (start 98 66) (end 98 65.434315) (width 0.5) (layer F.Cu) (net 10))
 (via (at 88 71) (size 0.8) (drill 0.4) (layers F.Cu B.Cu) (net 11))
 (segment (start 89.596 72.596) (end 88 71) (width 0.5) (layer F.Cu) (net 11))
 (segment (start 90.602 72.596) (end 89.596 72.596) (width 0.5) (layer F.Cu) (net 11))
 (segment (start 88 71) (end 93 66) (width 0.5) (layer B.Cu) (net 11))
 (via (at 98 64) (size 0.8) (drill 0.4) (layers F.Cu B.Cu) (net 11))
 (segment (start 96 66) (end 98 64) (width 0.5) (layer B.Cu) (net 11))
 (segment (start 93 66) (end 96 66) (width 0.5) (layer B.Cu) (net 11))
 (segment (start 97.325 63.325) (end 96.202 63.325) (width 0.5) (layer F.Cu) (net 11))
 (segment (start 98 64) (end 97.325 63.325) (width 0.5) (layer F.Cu) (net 11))
 (segment (start 86.686998 62.055) (end 88.902 62.055) (width 0.5) (layer F.Cu) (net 6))
 (segment (start 86.149999 62.591999) (end 86.686998 62.055) (width 0.5) (layer F.Cu) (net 6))
 (segment (start 86.149999 71.113999) (end 86.149999 62.591999) (width 0.5) (layer F.Cu) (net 6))
 (segment (start 88.902 73.866) (end 86.149999 71.113999) (width 0.5) (layer F.Cu) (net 6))
 (segment (start 90.602 73.866) (end 88.902 73.866) (width 0.5) (layer F.Cu) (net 6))
 (via (at 87 63) (size 0.8) (drill 0.4) (layers F.Cu B.Cu) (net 7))
 (segment (start 87.325 63.325) (end 87 63) (width 0.5) (layer F.Cu) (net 7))
 (segment (start 88.902 63.325) (end 87.325 63.325) (width 0.5) (layer F.Cu) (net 7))
 (segment (start 87 63) (end 87 61) (width 0.5) (layer B.Cu) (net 7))
 (segment (start 87 61) (end 89 59) (width 0.5) (layer B.Cu) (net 7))
 (segment (start 89 59) (end 97 59) (width 0.5) (layer B.Cu) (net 7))
 (segment (start 97 59) (end 99 61) (width 0.5) (layer B.Cu) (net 7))
 (segment (start 99 61) (end 104 66) (width 0.5) (layer B.Cu) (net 7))
 (via (at 104 66) (size 0.8) (drill 0.4) (layers F.Cu B.Cu) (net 7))
 (segment (start 107.538 71.4625) (end 106.4625 71.4625) (width 0.5) (layer F.Cu) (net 7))
 (segment (start 104 69) (end 104 66) (width 0.5) (layer F.Cu) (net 7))
 (segment (start 106.4625 71.4625) (end 104 69) (width 0.5) (layer F.Cu) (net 7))
 (segment (start 107.538 71.4625) (end 107.538 80) (width 0.5) (layer F.Cu) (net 7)))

